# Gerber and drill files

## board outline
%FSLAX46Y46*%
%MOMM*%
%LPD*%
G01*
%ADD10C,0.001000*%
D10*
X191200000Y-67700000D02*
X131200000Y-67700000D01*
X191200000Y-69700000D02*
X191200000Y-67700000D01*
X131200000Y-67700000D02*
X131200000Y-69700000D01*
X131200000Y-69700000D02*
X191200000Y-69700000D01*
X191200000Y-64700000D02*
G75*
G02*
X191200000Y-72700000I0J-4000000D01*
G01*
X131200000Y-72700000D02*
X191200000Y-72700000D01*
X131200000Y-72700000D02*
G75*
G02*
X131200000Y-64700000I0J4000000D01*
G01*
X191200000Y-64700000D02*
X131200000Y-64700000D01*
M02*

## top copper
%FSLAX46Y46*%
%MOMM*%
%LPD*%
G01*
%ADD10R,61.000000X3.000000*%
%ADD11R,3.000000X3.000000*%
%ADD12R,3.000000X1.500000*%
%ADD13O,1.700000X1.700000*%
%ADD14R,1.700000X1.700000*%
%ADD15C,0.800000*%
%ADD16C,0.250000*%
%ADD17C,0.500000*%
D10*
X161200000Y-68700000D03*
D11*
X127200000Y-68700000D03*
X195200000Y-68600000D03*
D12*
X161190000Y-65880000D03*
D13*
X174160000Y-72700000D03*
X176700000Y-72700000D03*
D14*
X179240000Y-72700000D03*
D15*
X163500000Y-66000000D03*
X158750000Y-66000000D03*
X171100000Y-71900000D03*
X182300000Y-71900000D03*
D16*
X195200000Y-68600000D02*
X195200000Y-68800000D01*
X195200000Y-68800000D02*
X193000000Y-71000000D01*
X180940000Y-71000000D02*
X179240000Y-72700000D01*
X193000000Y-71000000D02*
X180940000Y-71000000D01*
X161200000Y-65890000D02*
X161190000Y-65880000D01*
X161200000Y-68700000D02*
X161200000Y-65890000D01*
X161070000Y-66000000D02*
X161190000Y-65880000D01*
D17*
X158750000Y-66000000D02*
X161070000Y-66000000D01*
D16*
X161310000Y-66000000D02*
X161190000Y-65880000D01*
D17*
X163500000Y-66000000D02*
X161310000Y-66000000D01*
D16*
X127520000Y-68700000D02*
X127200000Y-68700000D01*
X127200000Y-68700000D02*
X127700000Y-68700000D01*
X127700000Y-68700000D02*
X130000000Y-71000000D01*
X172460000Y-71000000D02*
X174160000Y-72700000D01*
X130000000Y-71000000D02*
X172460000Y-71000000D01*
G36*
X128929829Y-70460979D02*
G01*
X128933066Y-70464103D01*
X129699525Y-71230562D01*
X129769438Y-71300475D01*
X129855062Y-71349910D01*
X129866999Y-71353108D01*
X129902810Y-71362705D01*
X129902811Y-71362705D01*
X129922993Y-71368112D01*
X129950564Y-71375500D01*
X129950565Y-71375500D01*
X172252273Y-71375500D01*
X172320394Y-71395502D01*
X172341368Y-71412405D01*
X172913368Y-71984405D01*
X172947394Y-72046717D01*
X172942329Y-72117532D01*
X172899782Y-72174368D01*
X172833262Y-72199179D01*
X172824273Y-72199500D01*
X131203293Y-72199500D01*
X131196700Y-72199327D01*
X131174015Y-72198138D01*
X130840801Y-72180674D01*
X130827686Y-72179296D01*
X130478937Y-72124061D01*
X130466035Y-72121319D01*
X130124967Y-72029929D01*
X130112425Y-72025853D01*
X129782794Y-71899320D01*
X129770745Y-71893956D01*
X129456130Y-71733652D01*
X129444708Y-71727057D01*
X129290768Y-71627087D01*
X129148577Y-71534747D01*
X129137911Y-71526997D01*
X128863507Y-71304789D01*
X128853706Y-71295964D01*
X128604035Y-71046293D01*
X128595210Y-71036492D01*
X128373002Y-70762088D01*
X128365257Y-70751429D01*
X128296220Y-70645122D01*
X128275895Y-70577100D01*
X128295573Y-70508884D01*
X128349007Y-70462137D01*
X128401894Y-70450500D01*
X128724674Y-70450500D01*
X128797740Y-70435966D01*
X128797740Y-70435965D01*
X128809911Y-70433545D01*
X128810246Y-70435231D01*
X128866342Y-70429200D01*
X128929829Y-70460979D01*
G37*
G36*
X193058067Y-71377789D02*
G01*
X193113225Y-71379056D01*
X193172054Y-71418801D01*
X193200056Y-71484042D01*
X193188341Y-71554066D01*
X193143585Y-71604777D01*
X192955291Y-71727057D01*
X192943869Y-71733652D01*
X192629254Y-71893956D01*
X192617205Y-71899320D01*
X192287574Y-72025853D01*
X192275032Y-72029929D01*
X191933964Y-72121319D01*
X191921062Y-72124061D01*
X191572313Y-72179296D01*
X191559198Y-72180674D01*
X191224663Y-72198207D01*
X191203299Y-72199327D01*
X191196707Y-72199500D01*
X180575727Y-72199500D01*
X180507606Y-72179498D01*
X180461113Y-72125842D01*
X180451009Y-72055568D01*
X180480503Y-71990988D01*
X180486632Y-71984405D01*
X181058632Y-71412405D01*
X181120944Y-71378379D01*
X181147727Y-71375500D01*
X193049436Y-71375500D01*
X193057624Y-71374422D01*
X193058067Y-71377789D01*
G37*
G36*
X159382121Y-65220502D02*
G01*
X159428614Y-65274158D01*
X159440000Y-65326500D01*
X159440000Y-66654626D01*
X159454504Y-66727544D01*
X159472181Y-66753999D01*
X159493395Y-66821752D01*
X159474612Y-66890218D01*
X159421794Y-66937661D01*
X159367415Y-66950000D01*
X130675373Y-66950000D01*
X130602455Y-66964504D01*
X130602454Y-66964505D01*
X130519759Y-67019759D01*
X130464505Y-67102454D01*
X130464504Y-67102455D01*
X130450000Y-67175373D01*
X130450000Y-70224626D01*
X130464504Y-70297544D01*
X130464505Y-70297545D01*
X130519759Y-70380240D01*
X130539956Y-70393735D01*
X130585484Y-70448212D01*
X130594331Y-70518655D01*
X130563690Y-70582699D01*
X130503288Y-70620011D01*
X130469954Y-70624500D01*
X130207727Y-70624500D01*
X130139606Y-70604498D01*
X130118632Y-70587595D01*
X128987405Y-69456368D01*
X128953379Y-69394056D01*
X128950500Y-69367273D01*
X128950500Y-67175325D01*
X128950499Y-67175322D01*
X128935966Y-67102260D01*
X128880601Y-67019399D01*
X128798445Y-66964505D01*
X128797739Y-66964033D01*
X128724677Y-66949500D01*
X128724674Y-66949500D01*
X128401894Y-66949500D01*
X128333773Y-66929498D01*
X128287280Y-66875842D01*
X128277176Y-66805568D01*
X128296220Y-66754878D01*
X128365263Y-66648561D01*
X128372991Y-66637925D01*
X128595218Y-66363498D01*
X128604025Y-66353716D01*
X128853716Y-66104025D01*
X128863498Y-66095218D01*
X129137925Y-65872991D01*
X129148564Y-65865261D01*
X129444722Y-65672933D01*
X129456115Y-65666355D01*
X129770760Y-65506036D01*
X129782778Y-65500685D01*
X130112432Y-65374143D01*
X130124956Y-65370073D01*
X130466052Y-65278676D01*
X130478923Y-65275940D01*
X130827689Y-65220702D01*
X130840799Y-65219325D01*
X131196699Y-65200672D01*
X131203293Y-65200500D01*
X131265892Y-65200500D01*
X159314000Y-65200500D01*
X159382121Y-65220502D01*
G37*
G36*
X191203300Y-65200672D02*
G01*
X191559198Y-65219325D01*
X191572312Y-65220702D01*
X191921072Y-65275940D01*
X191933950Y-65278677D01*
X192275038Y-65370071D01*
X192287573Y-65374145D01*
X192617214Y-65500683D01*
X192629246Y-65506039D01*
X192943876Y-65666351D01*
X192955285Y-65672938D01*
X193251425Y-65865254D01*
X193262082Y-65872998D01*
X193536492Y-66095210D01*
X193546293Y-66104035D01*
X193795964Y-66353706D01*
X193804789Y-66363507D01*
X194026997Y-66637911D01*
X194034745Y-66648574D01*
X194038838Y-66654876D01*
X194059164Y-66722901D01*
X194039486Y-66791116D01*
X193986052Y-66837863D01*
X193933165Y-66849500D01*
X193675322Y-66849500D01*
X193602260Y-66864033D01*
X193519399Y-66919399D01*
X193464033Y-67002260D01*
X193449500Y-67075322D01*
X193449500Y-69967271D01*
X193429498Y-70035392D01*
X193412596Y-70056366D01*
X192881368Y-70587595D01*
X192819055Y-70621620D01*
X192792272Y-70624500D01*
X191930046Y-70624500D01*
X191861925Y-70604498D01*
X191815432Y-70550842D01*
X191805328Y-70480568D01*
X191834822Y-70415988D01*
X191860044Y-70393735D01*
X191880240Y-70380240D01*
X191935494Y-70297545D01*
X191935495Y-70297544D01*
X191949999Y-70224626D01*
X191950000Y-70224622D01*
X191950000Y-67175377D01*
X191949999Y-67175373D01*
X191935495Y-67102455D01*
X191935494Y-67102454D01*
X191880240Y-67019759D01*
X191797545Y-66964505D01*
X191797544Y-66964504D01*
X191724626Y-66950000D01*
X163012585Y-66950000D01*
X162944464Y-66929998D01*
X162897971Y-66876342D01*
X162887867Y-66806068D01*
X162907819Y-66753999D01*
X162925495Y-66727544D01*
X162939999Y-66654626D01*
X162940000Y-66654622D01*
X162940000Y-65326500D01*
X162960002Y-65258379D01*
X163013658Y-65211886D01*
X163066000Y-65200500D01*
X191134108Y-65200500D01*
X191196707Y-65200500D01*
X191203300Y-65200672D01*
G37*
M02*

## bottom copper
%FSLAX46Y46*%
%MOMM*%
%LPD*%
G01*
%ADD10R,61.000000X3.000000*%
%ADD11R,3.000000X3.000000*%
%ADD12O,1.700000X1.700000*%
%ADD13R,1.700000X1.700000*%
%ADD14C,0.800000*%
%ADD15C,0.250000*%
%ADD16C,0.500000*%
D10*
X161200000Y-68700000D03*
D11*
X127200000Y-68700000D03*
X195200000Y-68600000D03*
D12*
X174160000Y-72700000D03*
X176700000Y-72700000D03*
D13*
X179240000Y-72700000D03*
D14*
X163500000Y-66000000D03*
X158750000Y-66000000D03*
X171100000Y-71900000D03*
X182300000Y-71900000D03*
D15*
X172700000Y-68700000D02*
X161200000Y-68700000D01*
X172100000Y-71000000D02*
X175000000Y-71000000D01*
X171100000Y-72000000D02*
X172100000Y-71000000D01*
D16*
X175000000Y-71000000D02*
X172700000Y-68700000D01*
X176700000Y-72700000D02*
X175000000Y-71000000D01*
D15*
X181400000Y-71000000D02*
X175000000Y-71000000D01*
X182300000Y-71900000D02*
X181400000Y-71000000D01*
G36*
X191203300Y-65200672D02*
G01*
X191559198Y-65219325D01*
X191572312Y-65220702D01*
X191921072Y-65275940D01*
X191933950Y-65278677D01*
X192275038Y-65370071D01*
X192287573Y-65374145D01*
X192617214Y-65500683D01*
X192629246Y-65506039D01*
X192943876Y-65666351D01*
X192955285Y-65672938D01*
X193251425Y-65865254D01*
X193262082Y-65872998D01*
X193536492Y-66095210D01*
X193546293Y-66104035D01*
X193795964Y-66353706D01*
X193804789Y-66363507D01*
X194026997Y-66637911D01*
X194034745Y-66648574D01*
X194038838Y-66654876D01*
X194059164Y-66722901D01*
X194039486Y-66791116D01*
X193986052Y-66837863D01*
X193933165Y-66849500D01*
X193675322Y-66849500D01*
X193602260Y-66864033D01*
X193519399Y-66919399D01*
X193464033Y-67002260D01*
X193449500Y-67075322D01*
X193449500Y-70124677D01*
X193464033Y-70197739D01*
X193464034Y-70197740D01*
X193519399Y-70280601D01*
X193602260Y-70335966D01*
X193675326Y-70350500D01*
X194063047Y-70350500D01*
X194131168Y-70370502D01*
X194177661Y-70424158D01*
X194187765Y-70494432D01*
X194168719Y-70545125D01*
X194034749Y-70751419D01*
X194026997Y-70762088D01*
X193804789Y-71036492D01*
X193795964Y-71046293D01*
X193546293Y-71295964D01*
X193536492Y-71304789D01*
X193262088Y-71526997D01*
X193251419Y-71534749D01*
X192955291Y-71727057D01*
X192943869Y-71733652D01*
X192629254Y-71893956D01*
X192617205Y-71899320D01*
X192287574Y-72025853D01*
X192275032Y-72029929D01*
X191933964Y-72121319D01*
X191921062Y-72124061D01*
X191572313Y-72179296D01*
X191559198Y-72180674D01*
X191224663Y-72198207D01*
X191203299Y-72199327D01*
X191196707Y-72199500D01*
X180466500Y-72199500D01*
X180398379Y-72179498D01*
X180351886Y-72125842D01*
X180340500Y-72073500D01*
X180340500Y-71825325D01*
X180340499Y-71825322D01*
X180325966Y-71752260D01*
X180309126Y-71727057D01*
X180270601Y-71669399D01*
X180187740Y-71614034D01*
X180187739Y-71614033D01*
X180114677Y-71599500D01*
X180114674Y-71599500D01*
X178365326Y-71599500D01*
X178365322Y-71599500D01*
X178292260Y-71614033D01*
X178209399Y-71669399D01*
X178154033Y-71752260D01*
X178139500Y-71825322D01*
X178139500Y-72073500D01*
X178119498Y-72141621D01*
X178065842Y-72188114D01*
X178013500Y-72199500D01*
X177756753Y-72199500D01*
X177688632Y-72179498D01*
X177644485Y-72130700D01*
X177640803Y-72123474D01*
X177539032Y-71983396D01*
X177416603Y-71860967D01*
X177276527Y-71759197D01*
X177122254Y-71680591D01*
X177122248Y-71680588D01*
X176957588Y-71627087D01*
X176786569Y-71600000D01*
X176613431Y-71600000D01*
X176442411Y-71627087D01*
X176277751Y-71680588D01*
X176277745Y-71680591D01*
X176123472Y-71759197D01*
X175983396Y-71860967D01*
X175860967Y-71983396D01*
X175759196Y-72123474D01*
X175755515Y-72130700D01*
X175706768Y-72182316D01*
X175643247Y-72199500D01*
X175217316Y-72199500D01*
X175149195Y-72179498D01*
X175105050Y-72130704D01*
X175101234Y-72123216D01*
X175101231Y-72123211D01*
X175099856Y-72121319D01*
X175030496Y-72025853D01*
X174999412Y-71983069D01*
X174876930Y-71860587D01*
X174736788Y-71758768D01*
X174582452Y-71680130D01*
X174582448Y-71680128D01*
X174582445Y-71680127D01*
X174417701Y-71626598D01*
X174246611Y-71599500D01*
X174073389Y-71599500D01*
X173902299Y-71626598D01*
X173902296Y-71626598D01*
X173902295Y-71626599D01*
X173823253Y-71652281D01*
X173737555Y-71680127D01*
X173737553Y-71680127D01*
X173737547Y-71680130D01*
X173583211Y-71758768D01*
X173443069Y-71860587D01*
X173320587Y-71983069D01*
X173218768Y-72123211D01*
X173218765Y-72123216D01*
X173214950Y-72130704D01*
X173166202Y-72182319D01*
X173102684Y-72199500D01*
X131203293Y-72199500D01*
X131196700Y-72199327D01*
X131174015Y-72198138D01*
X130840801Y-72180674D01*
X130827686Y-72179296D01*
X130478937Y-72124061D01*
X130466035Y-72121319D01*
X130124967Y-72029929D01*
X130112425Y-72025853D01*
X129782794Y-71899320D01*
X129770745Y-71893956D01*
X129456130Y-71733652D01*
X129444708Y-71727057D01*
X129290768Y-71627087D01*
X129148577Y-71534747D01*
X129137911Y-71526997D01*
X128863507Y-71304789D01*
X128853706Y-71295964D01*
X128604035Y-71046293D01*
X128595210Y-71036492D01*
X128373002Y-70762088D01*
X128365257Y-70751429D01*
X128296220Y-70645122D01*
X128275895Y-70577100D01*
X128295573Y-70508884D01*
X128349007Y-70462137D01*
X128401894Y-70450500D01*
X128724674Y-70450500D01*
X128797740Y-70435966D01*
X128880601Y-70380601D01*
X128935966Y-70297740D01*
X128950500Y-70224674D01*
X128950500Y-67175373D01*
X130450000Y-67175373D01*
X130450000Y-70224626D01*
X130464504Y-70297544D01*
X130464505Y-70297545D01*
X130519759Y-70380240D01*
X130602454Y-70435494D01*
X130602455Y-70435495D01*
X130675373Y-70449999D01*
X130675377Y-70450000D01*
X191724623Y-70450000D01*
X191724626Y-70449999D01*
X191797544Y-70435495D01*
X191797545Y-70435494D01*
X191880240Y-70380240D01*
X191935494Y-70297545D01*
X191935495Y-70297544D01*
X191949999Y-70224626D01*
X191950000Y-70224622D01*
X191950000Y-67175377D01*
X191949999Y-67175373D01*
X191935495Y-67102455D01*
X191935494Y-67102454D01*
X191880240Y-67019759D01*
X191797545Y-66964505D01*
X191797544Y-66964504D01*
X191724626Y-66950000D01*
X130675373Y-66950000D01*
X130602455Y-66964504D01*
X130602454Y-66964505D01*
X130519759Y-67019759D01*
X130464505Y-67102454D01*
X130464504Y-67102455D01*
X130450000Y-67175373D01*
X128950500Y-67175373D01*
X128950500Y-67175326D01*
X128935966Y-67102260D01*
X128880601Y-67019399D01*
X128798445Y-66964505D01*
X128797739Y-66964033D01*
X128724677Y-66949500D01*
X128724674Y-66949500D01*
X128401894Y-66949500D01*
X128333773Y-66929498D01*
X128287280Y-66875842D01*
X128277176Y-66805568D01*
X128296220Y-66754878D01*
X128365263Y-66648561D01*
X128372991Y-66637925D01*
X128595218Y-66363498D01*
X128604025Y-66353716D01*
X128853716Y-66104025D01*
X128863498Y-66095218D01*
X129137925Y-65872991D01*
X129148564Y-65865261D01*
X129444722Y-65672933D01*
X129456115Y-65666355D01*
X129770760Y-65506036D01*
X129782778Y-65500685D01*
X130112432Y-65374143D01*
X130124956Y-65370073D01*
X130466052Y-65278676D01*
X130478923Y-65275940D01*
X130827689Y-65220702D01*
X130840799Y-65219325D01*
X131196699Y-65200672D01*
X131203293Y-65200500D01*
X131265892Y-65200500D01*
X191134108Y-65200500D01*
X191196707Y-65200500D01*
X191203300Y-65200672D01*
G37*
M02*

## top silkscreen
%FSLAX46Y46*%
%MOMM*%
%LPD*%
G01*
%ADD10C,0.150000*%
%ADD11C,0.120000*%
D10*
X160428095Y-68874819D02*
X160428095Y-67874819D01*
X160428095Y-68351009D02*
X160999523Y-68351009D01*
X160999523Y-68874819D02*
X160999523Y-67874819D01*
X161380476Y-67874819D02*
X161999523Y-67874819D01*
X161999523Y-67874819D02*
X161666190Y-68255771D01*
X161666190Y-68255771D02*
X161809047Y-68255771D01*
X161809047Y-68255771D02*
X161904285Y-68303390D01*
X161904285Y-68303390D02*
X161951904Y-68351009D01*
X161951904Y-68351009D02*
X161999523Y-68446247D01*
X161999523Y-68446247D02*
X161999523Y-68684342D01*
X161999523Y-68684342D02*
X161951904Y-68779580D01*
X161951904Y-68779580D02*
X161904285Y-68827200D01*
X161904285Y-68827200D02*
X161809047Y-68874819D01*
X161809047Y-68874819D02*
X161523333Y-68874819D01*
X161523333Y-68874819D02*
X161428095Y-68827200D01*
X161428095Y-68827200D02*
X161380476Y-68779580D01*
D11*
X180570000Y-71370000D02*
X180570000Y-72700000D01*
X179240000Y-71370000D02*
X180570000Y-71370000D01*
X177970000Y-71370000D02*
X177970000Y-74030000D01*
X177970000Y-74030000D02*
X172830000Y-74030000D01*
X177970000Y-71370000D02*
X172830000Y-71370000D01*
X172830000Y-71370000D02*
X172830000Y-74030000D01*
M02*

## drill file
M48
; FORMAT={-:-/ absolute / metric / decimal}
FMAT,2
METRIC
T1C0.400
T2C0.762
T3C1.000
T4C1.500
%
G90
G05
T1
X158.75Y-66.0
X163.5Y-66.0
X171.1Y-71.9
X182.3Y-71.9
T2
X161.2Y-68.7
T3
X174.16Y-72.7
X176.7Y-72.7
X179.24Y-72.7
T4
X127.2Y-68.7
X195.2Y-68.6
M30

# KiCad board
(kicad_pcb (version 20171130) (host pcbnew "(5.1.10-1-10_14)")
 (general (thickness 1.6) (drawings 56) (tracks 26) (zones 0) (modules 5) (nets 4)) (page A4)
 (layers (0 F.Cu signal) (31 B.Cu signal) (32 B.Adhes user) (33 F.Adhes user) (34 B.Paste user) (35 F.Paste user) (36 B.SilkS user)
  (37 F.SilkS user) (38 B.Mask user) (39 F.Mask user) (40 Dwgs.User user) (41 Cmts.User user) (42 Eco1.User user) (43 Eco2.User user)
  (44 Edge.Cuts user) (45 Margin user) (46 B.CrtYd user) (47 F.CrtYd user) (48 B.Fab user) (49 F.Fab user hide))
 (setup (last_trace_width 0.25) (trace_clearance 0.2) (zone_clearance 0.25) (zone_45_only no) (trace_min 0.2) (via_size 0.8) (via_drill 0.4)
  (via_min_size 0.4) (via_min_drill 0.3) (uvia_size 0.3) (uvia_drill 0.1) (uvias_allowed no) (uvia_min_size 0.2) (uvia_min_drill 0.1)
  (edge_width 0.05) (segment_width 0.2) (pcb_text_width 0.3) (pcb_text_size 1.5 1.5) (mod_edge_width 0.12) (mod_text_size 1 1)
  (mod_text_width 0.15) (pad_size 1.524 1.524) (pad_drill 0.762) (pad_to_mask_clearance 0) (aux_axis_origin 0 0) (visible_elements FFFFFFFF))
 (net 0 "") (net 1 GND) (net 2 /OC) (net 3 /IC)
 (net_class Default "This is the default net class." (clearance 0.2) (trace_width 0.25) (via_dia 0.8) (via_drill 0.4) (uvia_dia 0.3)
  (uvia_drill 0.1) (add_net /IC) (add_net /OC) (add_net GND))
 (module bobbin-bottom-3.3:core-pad (layer F.Cu) (at 161.2 68.7)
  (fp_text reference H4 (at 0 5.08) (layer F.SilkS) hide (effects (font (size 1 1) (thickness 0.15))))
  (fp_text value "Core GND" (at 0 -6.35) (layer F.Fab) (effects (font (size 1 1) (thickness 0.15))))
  (pad 1 thru_hole rect (at 0 0) (size 61 3) (drill 0.762) (layers *.Cu *.Mask) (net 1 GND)))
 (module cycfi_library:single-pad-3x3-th (layer F.Cu) (at 127.2 68.7)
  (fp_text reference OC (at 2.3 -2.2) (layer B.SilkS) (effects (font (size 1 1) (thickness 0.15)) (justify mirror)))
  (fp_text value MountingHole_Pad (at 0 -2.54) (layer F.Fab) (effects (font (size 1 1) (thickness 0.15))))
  (pad 1 thru_hole rect (at 0 0) (size 3 3) (drill 1.5) (layers *.Cu *.Mask) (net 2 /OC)))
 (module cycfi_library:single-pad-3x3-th (layer F.Cu) (at 195.2 68.6)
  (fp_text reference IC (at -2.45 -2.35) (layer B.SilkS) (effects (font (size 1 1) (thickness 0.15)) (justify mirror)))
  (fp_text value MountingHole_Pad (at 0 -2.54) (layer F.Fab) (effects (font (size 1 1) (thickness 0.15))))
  (pad 1 thru_hole rect (at 0 0) (size 3 3) (drill 1.5) (layers *.Cu *.Mask) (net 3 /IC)))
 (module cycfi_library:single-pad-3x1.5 (layer F.Cu) (at 161.19 65.88)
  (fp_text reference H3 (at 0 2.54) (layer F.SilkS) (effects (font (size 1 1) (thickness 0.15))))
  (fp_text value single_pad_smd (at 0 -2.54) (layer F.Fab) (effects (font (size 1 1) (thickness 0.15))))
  (pad 1 smd rect (at 0 0) (size 3 1.5) (layers F.Cu F.Paste F.Mask) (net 1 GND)))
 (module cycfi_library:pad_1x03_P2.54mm (layer F.Cu) (at 179.24 72.7 270)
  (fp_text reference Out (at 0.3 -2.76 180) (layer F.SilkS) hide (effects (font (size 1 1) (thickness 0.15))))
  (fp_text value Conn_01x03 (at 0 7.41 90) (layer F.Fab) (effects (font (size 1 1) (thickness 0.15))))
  (fp_line (start -1.33 -1.33) (end 0 -1.33) (layer F.SilkS) (width 0.12))
  (fp_line (start -1.33 0) (end -1.33 -1.33) (layer F.SilkS) (width 0.12))
  (fp_line (start -1.33 1.27) (end 1.33 1.27) (layer F.SilkS) (width 0.12))
  (fp_line (start 1.33 1.27) (end 1.33 6.41) (layer F.SilkS) (width 0.12))
  (fp_line (start -1.33 1.27) (end -1.33 6.41) (layer F.SilkS) (width 0.12))
  (fp_line (start -1.33 6.41) (end 1.33 6.41) (layer F.SilkS) (width 0.12))
  (pad 3 thru_hole oval (at 0 5.08 270) (size 1.7 1.7) (drill 1) (layers *.Cu *.Mask) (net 2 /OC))
  (pad 2 thru_hole oval (at 0 2.54 270) (size 1.7 1.7) (drill 1) (layers *.Cu *.Mask) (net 1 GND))
  (pad 1 thru_hole rect (at 0 0 270) (size 1.7 1.7) (drill 1) (layers *.Cu *.Mask) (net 3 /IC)))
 (gr_line (start 191.2 67.7) (end 131.2 67.7) (layer Edge.Cuts) (width 0.001))
 (gr_line (start 191.2 69.7) (end 191.2 67.7) (layer Edge.Cuts) (width 0.001))
 (gr_line (start 131.2 67.7) (end 131.2 69.7) (layer Edge.Cuts) (width 0.001))
 (gr_line (start 131.2 69.7) (end 191.2 69.7) (layer Edge.Cuts) (width 0.001))
 (gr_arc (start 191.2 68.7) (end 191.2 72.7) (angle -180) (layer Edge.Cuts) (width 0.001))
 (gr_line (start 131.2 72.7) (end 191.2 72.7) (layer Edge.Cuts) (width 0.001))
 (gr_arc (start 131.2 68.7) (end 131.2 64.7) (angle -180) (layer Edge.Cuts) (width 0.001))
 (gr_line (start 191.2 64.7) (end 131.2 64.7) (layer Edge.Cuts) (width 0.001))
 (via (at 163.5 66) (size 0.8) (drill 0.4) (layers F.Cu B.Cu) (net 1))
 (via (at 158.75 66) (size 0.8) (drill 0.4) (layers F.Cu B.Cu) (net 1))
 (via (at 171.1 71.9) (size 0.8) (drill 0.4) (layers F.Cu B.Cu) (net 1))
 (via (at 182.3 71.9) (size 0.8) (drill 0.4) (layers F.Cu B.Cu) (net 1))
 (segment (start 195.2 68.6) (end 195.2 68.8) (width 0.25) (layer F.Cu) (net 3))
 (segment (start 195.2 68.8) (end 193 71) (width 0.25) (layer F.Cu) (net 3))
 (segment (start 180.94 71) (end 179.24 72.7) (width 0.25) (layer F.Cu) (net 3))
 (segment (start 193 71) (end 180.94 71) (width 0.25) (layer F.Cu) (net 3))
 (segment (start 161.2 65.89) (end 161.19 65.88) (width 0.25) (layer F.Cu) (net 1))
 (segment (start 161.2 68.7) (end 161.2 65.89) (width 0.25) (layer F.Cu) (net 1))
 (segment (start 172.7 68.7) (end 161.2 68.7) (width 0.25) (layer B.Cu) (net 1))
 (segment (start 172.1 71) (end 175 71) (width 0.25) (layer B.Cu) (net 1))
 (segment (start 171.1 72) (end 172.1 71) (width 0.25) (layer B.Cu) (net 1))
 (segment (start 175 71) (end 172.7 68.7) (width 0.5) (layer B.Cu) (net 1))
 (segment (start 176.7 72.7) (end 175 71) (width 0.5) (layer B.Cu) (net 1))
 (segment (start 181.4 71) (end 175 71) (width 0.25) (layer B.Cu) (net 1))
 (segment (start 182.3 71.9) (end 181.4 71) (width 0.25) (layer B.Cu) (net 1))
 (segment (start 161.07 66) (end 161.19 65.88) (width 0.25) (layer F.Cu) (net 1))
 (segment (start 158.75 66) (end 161.07 66) (width 0.5) (layer F.Cu) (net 1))
 (segment (start 161.31 66) (end 161.19 65.88) (width 0.25) (layer F.Cu) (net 1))
 (segment (start 163.5 66) (end 161.31 66) (width 0.5) (layer F.Cu) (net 1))
 (segment (start 127.52 68.7) (end 127.2 68.7) (width 0.25) (layer F.Cu) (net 2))
 (segment (start 127.2 68.7) (end 127.7 68.7) (width 0.25) (layer F.Cu) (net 2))
 (segment (start 127.7 68.7) (end 130 71) (width 0.25) (layer F.Cu) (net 2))
 (segment (start 172.46 71) (end 174.16 72.7) (width 0.25) (layer F.Cu) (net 2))
 (segment (start 130 71) (end 172.46 71) (width 0.25) (layer F.Cu) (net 2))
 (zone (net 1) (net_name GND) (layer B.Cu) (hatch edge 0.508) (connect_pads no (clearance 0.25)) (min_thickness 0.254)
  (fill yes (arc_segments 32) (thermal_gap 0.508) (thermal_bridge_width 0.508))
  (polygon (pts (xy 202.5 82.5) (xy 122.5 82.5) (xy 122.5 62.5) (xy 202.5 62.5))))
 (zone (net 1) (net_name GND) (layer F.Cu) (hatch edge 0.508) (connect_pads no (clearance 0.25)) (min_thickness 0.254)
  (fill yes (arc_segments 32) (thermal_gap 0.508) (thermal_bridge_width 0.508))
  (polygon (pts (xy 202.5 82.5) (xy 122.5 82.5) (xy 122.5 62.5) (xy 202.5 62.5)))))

